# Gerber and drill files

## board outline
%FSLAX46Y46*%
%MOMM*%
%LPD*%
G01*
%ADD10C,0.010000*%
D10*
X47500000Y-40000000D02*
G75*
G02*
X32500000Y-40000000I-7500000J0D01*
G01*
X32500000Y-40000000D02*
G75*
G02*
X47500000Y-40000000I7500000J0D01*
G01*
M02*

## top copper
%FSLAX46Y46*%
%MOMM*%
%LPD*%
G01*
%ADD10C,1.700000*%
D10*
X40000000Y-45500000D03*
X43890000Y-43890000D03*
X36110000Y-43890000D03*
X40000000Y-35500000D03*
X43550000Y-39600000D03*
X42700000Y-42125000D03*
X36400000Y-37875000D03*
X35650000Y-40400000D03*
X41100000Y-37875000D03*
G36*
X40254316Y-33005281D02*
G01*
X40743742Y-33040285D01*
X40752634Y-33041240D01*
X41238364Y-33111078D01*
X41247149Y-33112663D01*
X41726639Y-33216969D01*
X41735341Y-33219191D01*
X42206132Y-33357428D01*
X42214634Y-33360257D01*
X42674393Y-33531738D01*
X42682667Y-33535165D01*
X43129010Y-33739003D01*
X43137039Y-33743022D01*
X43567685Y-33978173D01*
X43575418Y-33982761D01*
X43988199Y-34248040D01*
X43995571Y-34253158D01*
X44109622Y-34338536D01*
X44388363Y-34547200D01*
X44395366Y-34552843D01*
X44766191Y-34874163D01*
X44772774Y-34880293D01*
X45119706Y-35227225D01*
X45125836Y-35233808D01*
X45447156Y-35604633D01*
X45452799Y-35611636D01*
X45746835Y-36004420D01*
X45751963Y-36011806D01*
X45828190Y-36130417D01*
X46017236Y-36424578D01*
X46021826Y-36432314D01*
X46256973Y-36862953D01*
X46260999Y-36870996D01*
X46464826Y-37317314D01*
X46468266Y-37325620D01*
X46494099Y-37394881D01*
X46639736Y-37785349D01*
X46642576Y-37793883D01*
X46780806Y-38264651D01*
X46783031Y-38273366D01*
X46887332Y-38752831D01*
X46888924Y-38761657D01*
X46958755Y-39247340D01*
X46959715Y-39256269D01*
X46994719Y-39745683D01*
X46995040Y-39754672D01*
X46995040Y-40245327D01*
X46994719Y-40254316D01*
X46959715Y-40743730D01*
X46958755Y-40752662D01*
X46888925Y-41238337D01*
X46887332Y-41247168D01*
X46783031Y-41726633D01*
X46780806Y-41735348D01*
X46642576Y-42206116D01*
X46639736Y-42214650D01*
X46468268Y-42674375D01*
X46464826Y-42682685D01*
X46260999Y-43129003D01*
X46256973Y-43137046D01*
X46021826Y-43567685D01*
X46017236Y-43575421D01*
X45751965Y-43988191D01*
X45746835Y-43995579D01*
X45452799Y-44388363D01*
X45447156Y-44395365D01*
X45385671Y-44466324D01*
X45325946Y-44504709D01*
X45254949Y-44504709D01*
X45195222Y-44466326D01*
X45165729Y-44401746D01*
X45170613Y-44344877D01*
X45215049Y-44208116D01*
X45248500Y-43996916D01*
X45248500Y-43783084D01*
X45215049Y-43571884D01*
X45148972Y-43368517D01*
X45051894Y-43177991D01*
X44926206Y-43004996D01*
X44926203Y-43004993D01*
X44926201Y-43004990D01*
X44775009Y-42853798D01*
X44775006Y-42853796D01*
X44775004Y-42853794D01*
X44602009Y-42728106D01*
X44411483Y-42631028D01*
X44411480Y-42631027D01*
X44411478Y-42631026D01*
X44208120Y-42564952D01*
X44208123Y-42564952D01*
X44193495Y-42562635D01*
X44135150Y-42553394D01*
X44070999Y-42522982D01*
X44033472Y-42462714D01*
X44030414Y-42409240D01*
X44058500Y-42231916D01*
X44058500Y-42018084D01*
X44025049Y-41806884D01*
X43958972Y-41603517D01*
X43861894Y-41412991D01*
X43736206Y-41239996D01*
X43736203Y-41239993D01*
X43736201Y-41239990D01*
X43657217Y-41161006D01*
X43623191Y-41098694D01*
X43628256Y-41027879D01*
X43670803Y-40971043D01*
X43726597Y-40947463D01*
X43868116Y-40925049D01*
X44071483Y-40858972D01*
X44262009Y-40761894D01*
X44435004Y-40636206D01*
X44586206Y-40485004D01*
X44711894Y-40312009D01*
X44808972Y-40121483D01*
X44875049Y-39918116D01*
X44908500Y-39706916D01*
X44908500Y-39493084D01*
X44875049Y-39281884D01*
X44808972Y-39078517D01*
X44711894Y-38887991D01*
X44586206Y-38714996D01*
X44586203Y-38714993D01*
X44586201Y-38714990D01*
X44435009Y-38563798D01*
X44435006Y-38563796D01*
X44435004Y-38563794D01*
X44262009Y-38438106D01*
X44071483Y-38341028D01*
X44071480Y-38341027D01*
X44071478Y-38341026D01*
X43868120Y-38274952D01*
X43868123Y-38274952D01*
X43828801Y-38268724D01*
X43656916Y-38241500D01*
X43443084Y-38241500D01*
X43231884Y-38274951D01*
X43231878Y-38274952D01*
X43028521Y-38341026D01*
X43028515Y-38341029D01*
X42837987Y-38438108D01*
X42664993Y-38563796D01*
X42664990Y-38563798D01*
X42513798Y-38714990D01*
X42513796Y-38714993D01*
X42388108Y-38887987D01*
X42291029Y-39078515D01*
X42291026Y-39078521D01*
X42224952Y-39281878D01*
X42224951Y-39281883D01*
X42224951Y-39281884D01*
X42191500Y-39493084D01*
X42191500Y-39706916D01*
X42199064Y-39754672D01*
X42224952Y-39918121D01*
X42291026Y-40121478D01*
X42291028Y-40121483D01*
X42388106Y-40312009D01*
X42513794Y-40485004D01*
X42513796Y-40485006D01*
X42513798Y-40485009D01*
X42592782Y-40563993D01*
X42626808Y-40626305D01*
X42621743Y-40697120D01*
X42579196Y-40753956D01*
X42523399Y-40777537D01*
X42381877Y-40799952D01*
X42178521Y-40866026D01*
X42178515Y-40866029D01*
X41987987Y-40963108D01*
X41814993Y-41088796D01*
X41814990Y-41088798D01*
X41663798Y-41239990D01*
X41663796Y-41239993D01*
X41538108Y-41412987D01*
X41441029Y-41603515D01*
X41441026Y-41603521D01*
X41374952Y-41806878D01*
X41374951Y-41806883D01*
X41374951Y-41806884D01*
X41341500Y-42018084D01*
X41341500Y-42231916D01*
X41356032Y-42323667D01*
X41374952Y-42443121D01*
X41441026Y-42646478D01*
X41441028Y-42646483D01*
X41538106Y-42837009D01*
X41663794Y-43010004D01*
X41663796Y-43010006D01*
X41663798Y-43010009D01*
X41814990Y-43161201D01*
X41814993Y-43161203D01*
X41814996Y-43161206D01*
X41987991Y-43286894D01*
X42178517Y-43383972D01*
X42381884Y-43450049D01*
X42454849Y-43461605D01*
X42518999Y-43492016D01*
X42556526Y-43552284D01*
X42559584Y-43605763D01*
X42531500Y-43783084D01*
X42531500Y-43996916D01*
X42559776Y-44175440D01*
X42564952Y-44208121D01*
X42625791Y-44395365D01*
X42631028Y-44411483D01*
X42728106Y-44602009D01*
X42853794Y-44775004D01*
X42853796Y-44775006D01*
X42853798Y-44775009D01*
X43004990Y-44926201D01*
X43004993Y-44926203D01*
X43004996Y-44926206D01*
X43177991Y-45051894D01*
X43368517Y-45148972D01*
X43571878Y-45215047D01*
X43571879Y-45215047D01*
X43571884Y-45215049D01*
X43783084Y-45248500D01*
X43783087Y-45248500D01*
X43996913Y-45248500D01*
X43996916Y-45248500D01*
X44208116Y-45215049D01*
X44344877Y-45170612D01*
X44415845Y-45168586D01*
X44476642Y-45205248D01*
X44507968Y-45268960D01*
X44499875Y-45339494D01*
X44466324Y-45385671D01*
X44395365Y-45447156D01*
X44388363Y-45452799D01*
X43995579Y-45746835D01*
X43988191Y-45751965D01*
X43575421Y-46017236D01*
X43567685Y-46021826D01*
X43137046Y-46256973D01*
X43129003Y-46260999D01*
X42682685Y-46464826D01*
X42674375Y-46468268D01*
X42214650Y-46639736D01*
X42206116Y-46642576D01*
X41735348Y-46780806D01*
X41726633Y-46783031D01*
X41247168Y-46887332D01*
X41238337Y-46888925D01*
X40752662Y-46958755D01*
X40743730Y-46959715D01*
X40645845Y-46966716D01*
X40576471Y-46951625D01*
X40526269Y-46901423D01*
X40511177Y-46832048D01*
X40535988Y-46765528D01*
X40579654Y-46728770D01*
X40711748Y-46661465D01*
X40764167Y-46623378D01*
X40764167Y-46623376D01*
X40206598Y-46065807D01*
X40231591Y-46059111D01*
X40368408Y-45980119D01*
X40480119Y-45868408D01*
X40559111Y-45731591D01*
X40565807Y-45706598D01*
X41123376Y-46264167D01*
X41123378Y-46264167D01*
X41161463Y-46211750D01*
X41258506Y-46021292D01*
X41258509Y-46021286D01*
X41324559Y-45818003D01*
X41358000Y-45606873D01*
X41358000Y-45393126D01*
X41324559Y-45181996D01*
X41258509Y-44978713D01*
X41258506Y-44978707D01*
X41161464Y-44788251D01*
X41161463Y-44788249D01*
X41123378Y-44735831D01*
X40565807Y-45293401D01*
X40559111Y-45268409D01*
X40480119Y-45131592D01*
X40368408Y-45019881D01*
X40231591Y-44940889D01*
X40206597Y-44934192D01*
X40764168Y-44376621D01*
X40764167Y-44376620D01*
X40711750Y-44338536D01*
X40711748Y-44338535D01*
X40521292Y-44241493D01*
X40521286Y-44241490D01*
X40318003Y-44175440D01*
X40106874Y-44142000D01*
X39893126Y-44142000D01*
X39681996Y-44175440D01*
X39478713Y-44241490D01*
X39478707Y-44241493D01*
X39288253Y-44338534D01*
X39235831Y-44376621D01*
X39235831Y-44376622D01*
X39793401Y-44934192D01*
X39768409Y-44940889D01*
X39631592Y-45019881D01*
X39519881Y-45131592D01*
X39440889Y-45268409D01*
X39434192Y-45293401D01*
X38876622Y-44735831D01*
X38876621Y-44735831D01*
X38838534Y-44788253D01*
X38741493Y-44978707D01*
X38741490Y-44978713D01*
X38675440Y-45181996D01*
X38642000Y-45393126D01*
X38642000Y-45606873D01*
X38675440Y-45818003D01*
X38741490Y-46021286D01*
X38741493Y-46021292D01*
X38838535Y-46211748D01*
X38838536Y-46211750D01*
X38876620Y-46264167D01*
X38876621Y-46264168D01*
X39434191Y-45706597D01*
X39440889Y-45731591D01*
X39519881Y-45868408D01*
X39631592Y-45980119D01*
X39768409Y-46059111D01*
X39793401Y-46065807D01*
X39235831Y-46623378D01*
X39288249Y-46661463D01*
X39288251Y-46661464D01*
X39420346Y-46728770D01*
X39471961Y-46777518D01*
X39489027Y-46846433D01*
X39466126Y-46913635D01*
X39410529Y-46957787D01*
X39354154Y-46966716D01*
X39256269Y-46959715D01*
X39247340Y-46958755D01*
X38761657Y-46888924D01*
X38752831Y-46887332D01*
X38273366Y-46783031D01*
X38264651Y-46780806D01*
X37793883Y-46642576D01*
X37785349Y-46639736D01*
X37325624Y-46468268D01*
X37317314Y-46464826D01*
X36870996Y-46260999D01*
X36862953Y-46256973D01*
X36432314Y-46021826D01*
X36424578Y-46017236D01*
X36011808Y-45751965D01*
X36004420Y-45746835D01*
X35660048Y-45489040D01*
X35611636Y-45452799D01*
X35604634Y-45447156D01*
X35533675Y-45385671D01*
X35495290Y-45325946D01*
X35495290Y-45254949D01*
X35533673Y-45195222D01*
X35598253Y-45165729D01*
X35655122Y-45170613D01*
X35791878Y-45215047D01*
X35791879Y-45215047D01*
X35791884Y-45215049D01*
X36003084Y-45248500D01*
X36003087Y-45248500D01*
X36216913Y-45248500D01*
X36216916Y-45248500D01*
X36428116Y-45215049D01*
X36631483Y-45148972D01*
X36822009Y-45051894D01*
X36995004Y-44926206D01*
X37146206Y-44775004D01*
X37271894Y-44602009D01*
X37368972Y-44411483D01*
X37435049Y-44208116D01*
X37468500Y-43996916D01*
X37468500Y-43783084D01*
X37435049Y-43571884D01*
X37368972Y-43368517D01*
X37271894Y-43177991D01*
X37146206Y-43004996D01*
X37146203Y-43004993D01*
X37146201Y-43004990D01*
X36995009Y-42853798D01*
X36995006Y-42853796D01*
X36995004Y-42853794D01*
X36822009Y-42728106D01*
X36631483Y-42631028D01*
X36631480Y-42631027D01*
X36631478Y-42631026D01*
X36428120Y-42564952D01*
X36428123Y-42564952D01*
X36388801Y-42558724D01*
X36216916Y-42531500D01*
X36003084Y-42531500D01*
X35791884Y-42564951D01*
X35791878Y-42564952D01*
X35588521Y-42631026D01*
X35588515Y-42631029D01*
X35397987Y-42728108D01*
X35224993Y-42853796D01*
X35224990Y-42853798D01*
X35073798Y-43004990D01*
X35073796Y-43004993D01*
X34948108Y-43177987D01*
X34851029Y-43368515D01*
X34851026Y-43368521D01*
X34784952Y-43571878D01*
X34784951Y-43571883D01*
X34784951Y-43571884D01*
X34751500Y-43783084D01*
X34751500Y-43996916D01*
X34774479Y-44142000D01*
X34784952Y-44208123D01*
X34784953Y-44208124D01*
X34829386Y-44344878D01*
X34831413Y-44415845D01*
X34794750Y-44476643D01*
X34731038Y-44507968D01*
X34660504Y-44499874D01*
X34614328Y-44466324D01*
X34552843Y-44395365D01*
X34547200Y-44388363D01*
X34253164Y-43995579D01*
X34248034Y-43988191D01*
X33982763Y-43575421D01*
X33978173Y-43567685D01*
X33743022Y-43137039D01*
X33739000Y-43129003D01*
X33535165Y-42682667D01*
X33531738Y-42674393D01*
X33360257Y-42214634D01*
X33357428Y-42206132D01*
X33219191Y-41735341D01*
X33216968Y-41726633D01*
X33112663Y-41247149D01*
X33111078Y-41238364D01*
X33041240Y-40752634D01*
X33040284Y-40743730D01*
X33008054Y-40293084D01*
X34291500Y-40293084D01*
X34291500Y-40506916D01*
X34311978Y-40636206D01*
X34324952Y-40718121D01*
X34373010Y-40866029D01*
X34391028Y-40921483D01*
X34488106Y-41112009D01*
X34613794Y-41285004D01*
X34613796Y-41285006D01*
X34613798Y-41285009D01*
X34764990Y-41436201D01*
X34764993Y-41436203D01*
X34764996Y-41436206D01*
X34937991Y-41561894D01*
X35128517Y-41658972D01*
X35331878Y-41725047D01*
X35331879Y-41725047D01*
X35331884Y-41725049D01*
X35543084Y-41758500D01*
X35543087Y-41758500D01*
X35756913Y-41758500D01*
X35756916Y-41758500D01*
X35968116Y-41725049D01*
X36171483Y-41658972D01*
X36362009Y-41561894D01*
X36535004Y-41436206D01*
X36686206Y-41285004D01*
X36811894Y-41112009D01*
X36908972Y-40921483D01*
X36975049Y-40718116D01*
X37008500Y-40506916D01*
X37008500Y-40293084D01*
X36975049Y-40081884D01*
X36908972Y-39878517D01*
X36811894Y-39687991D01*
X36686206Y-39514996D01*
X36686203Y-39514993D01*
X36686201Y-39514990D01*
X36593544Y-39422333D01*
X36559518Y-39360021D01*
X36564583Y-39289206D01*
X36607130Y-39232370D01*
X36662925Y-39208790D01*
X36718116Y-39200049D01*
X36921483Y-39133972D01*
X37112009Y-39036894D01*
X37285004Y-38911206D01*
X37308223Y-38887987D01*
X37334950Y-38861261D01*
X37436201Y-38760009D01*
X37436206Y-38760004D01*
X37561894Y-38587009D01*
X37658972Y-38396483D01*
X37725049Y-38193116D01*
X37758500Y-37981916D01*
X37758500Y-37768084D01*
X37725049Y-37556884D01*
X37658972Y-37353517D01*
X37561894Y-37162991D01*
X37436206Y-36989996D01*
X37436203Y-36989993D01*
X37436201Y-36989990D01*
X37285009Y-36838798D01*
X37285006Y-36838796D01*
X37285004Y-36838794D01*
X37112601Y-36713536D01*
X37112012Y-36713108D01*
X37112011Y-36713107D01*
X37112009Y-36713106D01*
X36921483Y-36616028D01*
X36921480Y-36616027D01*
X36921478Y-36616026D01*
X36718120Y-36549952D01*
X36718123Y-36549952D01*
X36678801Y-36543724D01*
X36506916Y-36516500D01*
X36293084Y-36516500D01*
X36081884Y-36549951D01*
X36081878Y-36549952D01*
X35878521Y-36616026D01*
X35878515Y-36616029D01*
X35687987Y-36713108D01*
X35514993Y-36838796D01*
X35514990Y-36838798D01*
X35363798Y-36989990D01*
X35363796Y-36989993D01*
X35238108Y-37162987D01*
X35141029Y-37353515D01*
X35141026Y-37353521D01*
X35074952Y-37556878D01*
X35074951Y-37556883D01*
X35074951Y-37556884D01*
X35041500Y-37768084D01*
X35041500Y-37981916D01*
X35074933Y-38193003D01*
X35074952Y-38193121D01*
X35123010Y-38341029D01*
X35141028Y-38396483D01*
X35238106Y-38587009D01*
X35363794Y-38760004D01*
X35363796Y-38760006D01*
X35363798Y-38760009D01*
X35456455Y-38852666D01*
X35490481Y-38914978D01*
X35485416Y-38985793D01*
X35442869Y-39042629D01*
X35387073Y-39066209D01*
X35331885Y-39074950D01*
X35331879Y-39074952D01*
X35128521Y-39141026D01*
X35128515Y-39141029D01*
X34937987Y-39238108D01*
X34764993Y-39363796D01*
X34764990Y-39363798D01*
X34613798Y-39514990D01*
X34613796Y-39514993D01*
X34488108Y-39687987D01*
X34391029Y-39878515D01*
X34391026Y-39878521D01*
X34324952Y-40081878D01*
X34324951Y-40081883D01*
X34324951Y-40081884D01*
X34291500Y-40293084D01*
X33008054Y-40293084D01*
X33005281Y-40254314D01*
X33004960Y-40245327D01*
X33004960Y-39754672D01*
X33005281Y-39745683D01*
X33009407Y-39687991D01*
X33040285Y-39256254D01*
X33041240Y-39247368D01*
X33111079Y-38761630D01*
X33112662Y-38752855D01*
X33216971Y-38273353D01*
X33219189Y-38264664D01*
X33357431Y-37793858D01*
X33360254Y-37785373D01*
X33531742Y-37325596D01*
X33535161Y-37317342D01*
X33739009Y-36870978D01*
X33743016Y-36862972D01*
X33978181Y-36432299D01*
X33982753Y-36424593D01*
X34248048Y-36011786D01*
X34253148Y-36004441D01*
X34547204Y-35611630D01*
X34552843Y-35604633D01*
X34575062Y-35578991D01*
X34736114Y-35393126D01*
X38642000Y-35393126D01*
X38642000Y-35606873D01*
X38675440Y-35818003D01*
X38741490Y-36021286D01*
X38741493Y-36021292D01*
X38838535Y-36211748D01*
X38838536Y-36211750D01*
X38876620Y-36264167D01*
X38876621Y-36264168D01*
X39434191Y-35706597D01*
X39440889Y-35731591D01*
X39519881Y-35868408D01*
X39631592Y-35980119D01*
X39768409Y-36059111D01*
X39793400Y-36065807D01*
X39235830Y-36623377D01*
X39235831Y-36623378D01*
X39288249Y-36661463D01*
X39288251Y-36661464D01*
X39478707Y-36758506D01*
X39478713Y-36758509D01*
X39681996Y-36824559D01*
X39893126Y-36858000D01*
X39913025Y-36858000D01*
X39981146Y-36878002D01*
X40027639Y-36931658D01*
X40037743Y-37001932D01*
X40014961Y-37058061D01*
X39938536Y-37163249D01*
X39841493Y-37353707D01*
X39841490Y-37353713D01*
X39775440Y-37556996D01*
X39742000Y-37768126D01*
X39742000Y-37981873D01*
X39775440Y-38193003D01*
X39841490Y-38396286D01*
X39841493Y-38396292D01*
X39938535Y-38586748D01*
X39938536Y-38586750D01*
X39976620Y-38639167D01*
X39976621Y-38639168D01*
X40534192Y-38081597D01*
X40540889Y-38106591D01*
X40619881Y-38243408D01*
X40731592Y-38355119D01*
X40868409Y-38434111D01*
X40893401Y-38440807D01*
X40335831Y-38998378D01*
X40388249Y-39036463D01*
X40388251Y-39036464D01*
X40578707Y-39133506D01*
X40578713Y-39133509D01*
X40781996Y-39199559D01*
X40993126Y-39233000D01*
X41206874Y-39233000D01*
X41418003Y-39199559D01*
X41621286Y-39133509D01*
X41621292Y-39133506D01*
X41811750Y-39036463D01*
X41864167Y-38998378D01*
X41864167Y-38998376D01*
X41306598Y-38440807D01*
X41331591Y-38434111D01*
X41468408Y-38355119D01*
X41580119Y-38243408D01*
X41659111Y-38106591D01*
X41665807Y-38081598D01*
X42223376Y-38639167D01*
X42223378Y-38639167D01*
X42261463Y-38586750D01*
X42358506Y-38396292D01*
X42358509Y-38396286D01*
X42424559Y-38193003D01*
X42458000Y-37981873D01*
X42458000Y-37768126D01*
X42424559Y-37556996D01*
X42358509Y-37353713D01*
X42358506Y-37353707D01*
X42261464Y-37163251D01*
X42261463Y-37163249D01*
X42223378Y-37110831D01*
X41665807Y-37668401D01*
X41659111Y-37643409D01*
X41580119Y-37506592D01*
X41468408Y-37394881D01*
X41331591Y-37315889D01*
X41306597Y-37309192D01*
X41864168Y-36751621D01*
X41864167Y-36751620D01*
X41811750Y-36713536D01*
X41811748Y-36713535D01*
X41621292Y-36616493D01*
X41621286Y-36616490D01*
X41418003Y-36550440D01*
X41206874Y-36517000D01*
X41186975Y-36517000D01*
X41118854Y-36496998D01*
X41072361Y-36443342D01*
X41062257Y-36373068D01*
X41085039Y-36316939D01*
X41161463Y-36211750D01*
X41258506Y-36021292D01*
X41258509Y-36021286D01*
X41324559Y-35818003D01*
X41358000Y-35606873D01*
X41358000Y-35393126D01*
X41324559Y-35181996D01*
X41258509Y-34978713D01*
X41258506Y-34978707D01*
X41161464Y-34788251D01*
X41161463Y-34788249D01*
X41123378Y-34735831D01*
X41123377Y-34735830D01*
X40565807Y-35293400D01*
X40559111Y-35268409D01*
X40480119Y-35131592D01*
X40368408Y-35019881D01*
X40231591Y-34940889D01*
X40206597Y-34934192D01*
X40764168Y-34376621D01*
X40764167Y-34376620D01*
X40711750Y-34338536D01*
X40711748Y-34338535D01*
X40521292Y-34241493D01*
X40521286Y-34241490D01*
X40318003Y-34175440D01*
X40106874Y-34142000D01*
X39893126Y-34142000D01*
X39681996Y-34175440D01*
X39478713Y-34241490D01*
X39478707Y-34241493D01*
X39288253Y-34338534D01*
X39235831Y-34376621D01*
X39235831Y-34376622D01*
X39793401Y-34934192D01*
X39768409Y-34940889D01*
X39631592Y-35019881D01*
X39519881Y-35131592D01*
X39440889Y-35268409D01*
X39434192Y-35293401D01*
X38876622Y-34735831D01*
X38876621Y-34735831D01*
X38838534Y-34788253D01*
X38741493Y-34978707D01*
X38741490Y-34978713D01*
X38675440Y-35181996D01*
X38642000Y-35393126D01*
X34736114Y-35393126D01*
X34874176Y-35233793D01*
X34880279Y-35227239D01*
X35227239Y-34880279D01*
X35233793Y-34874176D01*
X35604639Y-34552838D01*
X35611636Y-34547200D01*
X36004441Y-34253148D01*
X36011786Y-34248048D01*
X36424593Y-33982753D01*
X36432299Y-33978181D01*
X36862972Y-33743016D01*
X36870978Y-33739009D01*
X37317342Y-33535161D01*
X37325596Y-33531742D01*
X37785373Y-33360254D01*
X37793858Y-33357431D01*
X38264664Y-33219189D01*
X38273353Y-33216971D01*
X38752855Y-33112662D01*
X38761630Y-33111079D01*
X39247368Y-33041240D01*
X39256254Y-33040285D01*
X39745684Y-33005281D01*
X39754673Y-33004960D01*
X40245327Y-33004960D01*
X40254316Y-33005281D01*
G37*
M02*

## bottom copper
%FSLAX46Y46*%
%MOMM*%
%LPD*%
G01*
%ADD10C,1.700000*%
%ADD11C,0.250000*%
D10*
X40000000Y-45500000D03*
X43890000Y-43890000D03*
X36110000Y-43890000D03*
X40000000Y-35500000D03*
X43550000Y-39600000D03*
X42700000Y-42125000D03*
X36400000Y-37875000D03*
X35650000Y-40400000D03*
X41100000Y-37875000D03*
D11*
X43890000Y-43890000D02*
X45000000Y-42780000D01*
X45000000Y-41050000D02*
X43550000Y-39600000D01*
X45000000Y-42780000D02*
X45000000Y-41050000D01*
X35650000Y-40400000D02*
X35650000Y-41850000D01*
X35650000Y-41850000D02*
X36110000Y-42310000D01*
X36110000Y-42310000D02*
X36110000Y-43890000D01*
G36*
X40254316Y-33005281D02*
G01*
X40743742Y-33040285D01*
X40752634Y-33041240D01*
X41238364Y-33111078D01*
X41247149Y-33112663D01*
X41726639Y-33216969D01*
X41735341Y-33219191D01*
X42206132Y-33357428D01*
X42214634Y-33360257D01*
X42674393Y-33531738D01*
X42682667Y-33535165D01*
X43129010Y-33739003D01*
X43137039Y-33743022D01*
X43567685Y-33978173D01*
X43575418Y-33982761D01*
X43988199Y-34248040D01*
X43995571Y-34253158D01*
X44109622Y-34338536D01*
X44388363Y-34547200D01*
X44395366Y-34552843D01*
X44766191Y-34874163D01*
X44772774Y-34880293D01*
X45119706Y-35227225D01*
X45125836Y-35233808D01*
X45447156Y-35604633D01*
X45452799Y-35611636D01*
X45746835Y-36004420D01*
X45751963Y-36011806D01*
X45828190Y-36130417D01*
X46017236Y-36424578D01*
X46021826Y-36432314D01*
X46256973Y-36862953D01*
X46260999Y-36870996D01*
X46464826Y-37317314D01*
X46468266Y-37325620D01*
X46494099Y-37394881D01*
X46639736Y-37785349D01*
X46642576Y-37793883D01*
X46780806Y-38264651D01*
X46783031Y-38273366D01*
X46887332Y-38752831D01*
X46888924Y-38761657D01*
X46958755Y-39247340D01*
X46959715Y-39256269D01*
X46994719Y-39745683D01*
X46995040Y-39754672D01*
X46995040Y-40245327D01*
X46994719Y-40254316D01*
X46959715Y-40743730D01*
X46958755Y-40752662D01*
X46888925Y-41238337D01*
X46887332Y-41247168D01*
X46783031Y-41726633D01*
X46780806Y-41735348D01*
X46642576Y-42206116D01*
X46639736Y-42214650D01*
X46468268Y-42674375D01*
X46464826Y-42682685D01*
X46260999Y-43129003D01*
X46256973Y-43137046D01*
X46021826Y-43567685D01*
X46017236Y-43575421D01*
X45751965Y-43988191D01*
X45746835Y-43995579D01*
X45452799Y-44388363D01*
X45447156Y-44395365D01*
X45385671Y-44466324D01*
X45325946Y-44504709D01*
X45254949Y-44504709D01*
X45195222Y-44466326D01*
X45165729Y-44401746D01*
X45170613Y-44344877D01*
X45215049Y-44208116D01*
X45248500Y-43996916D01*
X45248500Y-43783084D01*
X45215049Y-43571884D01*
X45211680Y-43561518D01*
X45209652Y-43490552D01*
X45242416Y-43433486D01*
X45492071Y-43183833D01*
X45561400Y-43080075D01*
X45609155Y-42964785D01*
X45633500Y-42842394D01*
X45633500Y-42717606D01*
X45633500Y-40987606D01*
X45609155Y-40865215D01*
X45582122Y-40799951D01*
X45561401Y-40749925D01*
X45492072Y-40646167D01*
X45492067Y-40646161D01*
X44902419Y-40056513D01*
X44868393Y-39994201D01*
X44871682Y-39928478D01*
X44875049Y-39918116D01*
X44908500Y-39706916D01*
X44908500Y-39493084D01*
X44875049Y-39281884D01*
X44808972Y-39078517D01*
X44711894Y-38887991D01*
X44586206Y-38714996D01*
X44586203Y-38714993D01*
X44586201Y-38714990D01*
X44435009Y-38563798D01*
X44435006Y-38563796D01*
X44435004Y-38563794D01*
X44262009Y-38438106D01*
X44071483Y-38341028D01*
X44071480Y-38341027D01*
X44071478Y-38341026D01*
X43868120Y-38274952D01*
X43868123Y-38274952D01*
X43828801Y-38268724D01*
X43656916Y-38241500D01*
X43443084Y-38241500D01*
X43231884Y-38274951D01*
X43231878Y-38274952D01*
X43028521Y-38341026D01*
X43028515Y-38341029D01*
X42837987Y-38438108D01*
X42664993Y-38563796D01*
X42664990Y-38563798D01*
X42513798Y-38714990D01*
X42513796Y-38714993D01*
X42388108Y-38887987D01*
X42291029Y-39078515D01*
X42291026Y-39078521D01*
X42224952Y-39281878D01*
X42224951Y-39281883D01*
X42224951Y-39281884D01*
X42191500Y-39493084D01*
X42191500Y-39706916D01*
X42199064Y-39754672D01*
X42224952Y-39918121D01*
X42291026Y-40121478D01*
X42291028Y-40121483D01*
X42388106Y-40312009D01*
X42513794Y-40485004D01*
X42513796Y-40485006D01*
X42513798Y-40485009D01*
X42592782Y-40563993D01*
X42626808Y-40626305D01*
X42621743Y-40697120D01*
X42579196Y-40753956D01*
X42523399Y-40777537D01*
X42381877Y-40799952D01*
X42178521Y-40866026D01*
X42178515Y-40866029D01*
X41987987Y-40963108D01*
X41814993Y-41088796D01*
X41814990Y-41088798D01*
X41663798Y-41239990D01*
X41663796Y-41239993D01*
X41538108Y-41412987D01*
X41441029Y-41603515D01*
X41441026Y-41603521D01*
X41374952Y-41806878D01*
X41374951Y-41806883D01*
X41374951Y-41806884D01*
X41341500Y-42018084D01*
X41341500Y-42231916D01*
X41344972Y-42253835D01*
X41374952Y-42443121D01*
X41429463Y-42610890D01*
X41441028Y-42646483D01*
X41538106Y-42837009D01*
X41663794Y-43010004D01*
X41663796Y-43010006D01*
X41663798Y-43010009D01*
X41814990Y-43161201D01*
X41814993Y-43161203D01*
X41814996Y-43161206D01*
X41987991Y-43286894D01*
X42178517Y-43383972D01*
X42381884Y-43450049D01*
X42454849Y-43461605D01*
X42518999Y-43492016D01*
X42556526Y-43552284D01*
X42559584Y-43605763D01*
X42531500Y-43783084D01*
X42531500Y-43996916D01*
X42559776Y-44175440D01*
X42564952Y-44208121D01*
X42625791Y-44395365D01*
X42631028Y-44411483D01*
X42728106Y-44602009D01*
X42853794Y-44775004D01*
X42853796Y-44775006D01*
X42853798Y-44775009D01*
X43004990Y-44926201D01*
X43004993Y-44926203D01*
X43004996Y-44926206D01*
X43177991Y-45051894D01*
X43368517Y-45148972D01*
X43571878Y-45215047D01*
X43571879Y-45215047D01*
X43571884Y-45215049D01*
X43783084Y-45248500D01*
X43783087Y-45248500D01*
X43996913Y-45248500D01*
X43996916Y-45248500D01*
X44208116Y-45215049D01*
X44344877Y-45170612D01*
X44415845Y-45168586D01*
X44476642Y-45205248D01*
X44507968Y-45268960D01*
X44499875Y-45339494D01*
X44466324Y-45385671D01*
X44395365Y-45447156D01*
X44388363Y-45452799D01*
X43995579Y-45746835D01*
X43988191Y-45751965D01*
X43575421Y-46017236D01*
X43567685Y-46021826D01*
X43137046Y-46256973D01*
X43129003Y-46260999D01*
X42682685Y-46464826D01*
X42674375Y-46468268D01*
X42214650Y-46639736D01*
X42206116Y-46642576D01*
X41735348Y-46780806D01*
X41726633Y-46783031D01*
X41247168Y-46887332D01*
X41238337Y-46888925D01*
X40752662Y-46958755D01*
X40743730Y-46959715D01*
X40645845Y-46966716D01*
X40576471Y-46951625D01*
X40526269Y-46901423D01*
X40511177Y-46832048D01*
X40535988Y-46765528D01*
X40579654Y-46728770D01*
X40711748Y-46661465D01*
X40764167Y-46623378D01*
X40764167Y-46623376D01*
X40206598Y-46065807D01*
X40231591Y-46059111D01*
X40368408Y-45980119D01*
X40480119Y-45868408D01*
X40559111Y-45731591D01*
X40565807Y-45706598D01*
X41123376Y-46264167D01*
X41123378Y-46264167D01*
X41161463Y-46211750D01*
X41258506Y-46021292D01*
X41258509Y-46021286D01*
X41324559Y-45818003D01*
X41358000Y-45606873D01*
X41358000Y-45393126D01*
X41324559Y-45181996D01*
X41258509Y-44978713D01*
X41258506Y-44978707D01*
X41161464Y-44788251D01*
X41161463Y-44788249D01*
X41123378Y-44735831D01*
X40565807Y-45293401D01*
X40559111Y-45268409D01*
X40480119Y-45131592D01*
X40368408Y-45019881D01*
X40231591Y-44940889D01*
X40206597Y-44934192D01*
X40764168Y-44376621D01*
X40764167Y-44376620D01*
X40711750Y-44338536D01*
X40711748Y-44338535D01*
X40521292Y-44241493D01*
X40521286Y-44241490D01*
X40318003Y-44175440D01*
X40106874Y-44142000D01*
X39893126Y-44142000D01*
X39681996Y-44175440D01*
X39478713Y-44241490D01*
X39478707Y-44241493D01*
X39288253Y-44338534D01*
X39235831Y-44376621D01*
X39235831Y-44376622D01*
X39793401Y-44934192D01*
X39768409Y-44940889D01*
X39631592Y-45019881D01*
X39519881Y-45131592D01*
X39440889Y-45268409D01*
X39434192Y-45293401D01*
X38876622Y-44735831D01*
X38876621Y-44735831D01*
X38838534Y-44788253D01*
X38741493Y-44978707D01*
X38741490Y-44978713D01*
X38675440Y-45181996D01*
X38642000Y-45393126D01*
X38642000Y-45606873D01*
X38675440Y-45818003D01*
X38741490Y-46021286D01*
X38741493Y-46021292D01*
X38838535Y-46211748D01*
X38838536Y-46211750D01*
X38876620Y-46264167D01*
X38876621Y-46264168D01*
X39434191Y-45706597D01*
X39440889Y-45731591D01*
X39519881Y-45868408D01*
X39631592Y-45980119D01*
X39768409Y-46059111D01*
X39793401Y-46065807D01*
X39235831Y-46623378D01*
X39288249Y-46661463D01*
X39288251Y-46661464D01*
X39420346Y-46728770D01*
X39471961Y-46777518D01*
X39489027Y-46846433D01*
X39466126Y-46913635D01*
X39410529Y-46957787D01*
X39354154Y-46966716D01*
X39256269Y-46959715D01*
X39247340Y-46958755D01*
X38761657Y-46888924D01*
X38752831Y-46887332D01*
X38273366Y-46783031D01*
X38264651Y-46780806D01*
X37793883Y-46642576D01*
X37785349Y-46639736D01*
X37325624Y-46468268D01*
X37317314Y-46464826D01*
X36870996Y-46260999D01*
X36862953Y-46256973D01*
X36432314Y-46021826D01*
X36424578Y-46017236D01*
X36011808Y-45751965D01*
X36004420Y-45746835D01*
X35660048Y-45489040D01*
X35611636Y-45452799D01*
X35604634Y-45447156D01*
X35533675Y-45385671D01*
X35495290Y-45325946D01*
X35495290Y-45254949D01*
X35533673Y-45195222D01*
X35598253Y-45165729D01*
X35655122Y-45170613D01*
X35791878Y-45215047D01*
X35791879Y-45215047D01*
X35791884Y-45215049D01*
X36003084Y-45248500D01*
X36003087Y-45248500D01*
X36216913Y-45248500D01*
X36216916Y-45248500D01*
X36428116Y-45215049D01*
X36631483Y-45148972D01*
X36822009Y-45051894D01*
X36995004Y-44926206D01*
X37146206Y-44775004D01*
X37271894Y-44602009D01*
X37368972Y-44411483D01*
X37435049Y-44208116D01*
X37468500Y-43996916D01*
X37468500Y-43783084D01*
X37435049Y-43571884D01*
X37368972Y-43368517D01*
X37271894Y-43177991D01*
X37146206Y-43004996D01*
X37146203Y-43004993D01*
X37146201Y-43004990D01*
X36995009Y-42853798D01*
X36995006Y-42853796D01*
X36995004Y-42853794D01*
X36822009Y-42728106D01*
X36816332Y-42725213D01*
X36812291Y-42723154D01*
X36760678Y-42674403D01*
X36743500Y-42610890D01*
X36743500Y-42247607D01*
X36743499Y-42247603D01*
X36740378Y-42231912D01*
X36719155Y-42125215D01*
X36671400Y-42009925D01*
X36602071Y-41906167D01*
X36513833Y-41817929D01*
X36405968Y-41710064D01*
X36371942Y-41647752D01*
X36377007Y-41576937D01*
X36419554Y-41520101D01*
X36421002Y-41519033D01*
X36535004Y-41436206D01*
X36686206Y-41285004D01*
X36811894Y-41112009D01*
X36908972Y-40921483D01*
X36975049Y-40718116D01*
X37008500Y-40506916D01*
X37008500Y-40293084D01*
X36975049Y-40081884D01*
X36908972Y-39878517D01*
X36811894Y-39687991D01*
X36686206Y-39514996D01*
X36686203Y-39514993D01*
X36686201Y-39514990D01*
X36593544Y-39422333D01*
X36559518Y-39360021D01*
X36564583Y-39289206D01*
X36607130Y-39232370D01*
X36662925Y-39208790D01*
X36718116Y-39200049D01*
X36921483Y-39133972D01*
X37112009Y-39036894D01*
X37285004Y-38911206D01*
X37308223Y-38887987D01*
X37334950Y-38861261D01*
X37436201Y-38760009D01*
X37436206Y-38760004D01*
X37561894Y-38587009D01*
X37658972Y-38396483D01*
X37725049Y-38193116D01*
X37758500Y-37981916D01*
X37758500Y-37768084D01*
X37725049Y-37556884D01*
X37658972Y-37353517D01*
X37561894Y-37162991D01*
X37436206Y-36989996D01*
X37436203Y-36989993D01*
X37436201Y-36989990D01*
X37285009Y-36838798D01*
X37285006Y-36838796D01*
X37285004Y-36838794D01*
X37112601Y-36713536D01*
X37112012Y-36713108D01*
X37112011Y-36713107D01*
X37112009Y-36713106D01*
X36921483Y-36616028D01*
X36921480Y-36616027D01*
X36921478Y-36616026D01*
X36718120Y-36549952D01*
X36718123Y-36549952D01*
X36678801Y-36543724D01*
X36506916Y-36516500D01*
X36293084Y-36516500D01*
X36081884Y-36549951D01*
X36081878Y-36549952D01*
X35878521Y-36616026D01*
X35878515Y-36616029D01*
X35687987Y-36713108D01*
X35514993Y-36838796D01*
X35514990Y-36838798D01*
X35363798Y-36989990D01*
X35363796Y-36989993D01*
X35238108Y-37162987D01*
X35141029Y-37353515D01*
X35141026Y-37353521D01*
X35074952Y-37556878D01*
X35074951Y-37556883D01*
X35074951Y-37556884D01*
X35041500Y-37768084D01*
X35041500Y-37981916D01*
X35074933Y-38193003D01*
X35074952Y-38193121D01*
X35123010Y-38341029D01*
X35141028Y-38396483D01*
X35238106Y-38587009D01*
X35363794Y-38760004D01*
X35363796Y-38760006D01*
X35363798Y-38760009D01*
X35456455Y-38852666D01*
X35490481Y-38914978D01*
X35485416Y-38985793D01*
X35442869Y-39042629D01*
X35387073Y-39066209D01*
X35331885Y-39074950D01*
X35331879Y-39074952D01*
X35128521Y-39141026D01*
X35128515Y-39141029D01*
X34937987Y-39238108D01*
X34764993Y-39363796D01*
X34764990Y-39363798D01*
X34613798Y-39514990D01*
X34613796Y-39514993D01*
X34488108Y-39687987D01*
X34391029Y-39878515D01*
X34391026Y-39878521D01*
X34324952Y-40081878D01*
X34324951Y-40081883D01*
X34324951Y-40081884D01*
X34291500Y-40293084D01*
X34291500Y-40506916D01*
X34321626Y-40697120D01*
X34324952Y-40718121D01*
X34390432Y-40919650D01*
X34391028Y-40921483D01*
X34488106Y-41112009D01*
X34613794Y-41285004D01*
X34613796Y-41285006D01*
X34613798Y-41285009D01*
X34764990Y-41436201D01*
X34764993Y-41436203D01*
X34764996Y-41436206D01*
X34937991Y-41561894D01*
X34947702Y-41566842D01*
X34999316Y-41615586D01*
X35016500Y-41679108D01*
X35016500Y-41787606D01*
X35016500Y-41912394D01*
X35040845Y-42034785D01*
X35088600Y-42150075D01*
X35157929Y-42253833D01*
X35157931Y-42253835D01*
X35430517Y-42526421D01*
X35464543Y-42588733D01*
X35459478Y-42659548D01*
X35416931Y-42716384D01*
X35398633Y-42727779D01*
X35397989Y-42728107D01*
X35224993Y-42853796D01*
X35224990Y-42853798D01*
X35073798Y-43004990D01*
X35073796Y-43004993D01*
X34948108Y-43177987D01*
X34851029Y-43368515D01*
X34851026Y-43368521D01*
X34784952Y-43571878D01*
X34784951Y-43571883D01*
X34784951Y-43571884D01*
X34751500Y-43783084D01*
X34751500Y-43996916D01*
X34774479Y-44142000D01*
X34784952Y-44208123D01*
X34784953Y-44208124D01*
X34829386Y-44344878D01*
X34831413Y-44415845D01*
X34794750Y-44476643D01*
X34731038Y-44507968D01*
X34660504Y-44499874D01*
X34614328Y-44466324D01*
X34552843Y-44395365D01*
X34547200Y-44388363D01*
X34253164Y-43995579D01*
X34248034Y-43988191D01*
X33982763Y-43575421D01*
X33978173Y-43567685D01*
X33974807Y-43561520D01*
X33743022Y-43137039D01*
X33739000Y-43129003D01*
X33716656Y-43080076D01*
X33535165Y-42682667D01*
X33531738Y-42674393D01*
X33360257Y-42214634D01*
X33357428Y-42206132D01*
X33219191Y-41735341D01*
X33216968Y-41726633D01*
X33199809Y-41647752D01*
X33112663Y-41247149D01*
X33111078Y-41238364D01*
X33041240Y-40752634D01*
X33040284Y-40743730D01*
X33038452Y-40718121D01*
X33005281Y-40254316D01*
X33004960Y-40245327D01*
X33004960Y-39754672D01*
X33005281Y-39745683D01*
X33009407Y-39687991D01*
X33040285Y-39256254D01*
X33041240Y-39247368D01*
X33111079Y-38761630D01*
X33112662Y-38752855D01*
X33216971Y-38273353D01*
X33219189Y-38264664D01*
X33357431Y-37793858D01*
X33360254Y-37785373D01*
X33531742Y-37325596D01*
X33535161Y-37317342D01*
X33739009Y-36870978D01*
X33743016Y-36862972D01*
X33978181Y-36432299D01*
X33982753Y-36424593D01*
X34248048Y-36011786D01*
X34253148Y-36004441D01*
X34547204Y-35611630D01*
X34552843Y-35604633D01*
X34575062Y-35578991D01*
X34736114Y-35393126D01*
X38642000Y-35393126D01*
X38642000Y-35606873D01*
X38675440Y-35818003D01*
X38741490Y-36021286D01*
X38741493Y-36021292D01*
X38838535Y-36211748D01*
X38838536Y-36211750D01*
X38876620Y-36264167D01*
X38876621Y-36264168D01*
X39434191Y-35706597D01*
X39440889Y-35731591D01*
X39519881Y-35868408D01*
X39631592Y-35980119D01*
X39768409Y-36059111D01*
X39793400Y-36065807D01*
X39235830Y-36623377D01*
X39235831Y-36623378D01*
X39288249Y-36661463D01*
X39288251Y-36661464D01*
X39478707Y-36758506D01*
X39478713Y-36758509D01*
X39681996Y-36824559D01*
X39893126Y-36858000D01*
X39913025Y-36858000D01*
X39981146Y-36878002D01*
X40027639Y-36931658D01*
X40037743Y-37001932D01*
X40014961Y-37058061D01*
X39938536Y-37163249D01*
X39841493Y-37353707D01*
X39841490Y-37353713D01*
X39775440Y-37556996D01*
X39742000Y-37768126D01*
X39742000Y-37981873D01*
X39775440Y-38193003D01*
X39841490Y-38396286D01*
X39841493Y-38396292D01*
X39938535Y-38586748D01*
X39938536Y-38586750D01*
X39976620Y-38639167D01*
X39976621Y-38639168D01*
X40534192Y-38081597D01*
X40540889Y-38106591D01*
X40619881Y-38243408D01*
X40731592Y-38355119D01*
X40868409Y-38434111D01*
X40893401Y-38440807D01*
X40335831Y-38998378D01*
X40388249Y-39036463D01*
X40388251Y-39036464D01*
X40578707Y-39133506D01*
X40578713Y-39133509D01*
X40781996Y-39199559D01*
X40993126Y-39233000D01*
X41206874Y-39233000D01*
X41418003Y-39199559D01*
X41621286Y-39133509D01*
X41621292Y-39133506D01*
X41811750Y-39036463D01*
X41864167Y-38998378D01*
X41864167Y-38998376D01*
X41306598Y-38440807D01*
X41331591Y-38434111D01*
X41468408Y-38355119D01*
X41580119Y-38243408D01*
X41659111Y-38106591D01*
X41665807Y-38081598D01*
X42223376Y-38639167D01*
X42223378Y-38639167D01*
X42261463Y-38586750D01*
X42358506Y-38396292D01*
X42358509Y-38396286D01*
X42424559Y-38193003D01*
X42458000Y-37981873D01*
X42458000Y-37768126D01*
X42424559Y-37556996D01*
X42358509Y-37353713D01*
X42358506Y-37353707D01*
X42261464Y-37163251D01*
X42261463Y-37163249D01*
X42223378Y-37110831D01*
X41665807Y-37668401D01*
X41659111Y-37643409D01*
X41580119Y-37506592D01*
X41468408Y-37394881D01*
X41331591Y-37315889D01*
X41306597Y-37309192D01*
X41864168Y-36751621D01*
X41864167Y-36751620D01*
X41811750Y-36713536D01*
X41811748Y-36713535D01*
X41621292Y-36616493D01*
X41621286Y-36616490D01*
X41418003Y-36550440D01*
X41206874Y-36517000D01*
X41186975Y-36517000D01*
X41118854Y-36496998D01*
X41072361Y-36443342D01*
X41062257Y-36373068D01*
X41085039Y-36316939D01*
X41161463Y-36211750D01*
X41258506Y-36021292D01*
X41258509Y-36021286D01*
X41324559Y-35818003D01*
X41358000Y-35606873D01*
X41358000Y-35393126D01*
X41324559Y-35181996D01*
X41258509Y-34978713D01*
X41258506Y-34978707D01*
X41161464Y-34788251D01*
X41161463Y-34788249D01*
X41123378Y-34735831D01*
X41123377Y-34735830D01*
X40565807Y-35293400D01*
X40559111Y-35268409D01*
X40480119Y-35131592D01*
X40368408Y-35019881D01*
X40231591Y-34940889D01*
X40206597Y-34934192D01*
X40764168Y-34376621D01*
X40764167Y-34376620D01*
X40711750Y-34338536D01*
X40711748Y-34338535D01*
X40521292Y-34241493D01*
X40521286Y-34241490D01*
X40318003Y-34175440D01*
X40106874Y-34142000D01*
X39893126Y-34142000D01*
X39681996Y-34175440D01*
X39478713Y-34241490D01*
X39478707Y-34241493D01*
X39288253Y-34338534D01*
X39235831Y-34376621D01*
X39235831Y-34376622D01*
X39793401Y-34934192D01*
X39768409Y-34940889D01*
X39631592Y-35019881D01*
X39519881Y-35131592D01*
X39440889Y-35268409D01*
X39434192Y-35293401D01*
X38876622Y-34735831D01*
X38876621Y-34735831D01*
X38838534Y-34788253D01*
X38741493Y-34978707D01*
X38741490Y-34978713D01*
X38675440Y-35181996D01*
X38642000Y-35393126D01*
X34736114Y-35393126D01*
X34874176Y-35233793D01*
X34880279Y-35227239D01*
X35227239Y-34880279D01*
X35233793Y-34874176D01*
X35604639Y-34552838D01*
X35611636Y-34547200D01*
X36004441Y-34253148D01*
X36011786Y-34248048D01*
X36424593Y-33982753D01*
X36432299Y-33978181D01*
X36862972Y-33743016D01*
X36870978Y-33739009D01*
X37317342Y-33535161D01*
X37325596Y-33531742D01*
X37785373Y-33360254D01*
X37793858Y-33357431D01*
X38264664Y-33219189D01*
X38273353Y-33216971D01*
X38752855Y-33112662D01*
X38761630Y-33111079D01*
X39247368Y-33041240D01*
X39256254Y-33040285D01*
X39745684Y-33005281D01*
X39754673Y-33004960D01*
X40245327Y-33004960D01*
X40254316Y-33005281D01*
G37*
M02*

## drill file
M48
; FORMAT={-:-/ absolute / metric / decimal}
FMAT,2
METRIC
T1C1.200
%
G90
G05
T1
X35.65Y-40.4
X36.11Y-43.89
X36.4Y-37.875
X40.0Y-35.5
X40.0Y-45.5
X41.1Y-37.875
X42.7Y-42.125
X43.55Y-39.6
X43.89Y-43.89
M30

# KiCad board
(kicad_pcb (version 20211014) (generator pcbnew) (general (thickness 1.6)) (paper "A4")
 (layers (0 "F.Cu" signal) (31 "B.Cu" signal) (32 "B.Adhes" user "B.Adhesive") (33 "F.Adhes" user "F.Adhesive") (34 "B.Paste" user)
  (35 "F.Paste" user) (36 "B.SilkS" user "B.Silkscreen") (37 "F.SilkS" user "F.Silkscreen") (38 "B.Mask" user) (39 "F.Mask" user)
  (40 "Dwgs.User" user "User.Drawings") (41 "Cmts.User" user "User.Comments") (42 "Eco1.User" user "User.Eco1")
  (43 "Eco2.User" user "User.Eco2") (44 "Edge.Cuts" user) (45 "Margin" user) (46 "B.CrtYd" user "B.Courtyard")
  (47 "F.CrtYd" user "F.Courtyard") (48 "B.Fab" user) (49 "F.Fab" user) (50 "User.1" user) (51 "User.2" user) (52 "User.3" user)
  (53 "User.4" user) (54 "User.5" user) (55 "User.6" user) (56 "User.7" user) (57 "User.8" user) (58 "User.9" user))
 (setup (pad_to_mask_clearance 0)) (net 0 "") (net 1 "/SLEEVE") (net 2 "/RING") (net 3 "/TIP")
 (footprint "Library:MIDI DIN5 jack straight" (layer "F.Cu") (at 40 40)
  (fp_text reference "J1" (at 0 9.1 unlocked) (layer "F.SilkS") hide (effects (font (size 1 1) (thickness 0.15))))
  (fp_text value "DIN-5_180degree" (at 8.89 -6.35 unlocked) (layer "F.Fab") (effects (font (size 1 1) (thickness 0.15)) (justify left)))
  (pad "2" thru_hole circle (at 0 5.5) (size 1.7 1.7) (drill 1.2) (layers *.Cu *.Mask) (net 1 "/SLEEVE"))
  (pad "4" thru_hole circle (at 3.89 3.89) (size 1.7 1.7) (drill 1.2) (layers *.Cu *.Mask) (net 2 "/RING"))
  (pad "5" thru_hole circle (at -3.89 3.89) (size 1.7 1.7) (drill 1.2) (layers *.Cu *.Mask) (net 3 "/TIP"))
  (pad "S" thru_hole circle (at 0 -4.5) (size 1.7 1.7) (drill 1.2) (layers *.Cu *.Mask) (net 1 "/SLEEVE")))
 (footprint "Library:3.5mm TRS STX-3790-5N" (layer "F.Cu") (at 40 40)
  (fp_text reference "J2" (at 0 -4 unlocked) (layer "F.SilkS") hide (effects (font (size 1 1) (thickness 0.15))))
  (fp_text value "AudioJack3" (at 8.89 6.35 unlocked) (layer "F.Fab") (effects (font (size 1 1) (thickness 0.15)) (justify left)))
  (pad "1" thru_hole circle (at 3.55 -0.4) (size 1.7 1.7) (drill 1.2) (layers *.Cu *.Mask) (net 2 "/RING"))
  (pad "2" thru_hole circle (at 2.7 2.125) (size 1.7 1.7) (drill 1.2) (layers *.Cu *.Mask))
  (pad "3" thru_hole circle (at -3.6 -2.125) (size 1.7 1.7) (drill 1.2) (layers *.Cu *.Mask))
  (pad "4" thru_hole circle (at -4.35 0.4) (size 1.7 1.7) (drill 1.2) (layers *.Cu *.Mask) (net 3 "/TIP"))
  (pad "5" thru_hole circle (at 1.1 -2.125) (size 1.7 1.7) (drill 1.2) (layers *.Cu *.Mask) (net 1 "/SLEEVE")))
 (gr_circle (center 40 40) (end 47.5 40) (layer "Edge.Cuts") (width 0.01) (fill none))
 (segment (start 43.89 43.89) (end 45 42.78) (width 0.25) (layer "B.Cu") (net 2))
 (segment (start 45 41.05) (end 43.55 39.6) (width 0.25) (layer "B.Cu") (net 2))
 (segment (start 45 42.78) (end 45 41.05) (width 0.25) (layer "B.Cu") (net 2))
 (segment (start 35.65 40.4) (end 35.65 41.85) (width 0.25) (layer "B.Cu") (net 3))
 (segment (start 35.65 41.85) (end 36.11 42.31) (width 0.25) (layer "B.Cu") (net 3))
 (segment (start 36.11 42.31) (end 36.11 43.89) (width 0.25) (layer "B.Cu") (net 3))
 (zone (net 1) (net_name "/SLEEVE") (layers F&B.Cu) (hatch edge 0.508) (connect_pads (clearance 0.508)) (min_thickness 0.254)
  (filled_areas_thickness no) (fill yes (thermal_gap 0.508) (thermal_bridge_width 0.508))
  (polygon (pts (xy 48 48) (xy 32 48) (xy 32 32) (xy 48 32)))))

